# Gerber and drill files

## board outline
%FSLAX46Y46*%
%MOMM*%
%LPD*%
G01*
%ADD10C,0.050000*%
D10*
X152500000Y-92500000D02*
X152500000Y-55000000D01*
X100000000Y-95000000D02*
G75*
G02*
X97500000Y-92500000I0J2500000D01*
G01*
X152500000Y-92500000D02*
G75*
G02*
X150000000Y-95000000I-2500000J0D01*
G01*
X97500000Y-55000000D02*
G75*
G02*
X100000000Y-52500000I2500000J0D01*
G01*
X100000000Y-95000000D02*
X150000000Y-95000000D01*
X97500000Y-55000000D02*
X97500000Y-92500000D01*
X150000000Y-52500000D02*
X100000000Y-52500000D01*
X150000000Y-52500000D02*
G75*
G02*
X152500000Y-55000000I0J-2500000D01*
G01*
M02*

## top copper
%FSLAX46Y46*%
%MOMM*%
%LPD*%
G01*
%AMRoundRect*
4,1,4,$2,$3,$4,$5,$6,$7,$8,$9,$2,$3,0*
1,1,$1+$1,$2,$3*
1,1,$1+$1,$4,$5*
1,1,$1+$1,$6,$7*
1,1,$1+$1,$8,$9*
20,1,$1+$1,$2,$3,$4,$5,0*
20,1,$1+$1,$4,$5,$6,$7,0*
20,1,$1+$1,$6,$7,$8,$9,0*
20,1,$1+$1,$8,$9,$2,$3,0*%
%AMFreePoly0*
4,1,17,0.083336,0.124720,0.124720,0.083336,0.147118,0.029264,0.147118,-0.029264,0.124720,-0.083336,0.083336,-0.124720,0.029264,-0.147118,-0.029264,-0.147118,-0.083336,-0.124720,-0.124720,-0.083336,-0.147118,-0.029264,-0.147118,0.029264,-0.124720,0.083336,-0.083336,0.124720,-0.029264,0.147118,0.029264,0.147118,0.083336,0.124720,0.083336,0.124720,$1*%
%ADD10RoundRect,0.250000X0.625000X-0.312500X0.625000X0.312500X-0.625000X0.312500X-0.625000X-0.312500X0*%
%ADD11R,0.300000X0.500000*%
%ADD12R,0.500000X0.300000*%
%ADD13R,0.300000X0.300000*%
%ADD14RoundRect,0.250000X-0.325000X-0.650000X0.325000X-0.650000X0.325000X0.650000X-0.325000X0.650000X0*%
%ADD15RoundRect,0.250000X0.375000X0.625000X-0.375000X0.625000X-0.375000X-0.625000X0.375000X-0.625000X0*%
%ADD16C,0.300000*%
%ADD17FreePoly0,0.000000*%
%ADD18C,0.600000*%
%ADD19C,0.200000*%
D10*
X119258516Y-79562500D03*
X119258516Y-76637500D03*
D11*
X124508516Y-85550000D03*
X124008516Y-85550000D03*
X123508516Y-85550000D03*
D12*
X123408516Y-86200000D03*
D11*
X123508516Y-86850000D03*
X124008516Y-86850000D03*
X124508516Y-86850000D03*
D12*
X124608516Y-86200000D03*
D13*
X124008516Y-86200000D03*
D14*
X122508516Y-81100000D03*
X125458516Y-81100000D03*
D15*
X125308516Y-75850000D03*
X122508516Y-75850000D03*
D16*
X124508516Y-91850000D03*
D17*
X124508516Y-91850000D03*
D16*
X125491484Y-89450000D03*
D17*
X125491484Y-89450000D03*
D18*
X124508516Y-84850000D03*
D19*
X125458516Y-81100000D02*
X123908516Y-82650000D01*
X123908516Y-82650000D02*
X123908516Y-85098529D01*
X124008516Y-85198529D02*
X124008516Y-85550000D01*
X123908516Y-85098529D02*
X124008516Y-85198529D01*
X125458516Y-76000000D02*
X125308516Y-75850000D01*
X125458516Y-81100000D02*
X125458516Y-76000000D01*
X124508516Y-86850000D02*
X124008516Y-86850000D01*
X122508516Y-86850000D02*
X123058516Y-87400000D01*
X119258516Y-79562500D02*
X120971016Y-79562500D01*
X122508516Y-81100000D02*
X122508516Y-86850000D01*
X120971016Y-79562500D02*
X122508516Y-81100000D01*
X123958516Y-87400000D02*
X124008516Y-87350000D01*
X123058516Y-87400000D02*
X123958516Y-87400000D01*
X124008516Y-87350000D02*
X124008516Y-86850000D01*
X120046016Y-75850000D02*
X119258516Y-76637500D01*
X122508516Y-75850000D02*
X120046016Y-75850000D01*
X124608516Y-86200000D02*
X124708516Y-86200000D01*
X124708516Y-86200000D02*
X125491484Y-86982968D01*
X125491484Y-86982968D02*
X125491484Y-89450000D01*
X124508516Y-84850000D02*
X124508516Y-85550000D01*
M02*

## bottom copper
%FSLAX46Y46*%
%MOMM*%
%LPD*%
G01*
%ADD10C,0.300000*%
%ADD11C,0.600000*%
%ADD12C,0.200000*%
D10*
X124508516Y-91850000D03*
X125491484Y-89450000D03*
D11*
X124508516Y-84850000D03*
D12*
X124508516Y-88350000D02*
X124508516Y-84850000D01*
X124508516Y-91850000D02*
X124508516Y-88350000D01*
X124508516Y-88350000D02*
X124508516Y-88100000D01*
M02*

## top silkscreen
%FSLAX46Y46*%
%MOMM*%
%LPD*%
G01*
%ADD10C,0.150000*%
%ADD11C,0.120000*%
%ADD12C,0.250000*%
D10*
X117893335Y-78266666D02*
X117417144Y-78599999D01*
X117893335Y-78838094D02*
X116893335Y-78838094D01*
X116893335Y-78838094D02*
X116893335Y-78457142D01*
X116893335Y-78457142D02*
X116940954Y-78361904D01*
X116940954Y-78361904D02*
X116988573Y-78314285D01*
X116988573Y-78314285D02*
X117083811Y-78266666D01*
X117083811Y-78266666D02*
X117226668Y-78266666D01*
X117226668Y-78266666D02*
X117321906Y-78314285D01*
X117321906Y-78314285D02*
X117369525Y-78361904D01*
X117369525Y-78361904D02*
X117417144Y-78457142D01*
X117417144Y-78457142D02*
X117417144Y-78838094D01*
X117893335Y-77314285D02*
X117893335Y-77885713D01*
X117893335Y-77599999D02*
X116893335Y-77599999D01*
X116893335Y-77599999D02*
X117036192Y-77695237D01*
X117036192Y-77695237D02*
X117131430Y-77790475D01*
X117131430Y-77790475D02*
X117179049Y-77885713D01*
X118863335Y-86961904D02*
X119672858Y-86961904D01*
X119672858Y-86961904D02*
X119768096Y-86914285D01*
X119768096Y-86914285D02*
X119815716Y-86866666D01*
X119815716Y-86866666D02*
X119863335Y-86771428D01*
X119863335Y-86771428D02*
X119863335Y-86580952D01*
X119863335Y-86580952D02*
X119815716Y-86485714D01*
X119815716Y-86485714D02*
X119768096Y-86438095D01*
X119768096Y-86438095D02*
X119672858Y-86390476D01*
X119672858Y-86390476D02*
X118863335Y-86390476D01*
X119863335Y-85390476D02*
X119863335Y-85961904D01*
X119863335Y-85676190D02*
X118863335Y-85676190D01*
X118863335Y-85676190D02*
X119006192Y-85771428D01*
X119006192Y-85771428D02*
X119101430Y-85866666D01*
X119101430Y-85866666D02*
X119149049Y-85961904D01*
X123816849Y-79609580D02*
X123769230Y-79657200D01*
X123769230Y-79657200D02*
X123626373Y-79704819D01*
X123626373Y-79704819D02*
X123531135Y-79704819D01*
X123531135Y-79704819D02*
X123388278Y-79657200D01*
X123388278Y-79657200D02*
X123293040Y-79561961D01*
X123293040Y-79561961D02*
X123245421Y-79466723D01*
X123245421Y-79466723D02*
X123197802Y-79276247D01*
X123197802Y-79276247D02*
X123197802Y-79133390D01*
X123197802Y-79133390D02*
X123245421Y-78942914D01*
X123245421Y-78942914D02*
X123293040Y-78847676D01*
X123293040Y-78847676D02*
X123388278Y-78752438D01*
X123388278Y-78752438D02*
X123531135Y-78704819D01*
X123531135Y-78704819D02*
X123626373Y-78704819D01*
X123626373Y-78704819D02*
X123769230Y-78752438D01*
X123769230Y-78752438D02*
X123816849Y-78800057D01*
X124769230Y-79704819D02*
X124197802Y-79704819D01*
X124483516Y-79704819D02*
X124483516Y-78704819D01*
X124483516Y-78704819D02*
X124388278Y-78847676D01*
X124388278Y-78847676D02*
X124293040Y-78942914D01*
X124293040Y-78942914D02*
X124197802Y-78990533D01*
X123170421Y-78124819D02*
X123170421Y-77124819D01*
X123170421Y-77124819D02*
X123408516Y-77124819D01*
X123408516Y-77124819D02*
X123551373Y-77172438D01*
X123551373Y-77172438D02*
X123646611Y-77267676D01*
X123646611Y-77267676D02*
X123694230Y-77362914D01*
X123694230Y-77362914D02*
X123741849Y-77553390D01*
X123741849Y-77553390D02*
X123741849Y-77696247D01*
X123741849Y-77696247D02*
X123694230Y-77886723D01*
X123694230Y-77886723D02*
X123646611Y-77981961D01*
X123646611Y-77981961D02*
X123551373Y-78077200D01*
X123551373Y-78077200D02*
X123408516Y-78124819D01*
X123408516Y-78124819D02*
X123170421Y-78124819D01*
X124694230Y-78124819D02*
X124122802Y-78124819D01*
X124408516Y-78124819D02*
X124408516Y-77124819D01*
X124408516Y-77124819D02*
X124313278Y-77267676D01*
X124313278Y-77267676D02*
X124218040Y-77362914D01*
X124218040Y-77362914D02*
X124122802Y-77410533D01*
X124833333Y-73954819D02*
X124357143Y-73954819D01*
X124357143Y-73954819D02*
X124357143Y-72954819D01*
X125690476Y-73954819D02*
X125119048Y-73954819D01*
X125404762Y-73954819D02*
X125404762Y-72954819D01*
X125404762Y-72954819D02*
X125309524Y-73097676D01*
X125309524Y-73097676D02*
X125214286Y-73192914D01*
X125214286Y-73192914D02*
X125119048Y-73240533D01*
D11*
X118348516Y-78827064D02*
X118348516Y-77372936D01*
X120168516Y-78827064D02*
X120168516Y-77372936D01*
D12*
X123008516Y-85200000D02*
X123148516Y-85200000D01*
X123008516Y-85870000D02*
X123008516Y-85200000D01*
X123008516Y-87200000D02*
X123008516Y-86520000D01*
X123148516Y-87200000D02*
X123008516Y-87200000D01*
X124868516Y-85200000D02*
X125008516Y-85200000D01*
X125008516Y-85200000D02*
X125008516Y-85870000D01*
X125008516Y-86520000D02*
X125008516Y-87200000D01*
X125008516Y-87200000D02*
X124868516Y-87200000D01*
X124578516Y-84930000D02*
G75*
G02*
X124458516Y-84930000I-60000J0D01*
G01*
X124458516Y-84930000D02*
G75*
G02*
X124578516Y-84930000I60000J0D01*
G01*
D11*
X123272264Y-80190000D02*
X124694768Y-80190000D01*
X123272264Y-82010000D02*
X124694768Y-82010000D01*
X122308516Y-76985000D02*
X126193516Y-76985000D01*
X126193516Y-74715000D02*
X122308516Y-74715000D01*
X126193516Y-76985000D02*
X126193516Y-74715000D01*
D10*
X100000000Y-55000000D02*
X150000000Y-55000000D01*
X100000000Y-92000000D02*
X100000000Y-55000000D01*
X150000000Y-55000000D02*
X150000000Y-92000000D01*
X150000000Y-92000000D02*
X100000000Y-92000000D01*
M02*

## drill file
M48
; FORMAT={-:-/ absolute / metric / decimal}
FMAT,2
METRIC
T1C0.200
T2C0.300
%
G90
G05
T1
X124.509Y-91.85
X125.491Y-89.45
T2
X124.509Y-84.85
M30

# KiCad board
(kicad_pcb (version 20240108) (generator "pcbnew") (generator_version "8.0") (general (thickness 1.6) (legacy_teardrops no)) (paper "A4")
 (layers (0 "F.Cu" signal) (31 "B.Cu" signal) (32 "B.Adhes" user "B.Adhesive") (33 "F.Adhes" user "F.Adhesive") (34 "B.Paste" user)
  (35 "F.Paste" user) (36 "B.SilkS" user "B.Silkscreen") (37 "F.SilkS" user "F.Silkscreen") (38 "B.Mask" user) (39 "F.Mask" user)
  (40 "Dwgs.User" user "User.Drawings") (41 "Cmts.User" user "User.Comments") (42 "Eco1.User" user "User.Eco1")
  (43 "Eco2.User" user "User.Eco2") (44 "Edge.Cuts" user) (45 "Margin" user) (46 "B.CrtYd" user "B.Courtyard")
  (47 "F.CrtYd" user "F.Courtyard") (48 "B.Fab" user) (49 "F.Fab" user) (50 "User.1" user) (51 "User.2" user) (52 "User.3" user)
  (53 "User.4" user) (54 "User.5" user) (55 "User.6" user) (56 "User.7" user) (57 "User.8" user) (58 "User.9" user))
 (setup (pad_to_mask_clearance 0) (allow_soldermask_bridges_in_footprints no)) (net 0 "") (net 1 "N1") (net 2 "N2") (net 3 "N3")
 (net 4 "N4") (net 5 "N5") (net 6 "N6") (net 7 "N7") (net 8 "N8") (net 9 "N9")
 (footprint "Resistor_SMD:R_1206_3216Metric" (layer "F.Cu") (at 119.258516 78.1 90)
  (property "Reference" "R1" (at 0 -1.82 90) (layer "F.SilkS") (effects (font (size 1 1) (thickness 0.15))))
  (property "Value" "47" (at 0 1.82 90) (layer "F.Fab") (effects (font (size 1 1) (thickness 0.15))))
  (fp_line (start -0.727064 -0.91) (end 0.727064 -0.91) (stroke (width 0.12) (type solid)) (layer "F.SilkS"))
  (fp_line (start -0.727064 0.91) (end 0.727064 0.91) (stroke (width 0.12) (type solid)) (layer "F.SilkS"))
  (pad "1" smd roundrect (at -1.4625 0 90) (size 1.125 1.75) (layers "F.Cu" "F.Paste" "F.Mask") (roundrect_rratio 0.222222) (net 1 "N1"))
  (pad "2" smd roundrect (at 1.4625 0 90) (size 1.125 1.75) (layers "F.Cu" "F.Paste" "F.Mask") (roundrect_rratio 0.222222) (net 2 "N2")))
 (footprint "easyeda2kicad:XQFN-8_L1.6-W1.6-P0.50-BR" (layer "F.Cu") (at 124.008516 86.2 90)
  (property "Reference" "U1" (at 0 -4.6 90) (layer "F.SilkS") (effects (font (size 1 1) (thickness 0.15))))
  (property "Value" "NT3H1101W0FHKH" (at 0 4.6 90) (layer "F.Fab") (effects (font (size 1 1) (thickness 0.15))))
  (fp_line (start 1 -1) (end 1 -0.86) (stroke (width 0.25) (type solid)) (layer "F.SilkS"))
  (fp_line (start 0.33 -1) (end 1 -1) (stroke (width 0.25) (type solid)) (layer "F.SilkS"))
  (fp_line (start -1 -1) (end -0.32 -1) (stroke (width 0.25) (type solid)) (layer "F.SilkS"))
  (fp_line (start -1 -0.86) (end -1 -1) (stroke (width 0.25) (type solid)) (layer "F.SilkS"))
  (fp_line (start 1 0.86) (end 1 1) (stroke (width 0.25) (type solid)) (layer "F.SilkS"))
  (fp_line (start 1 1) (end 0.33 1) (stroke (width 0.25) (type solid)) (layer "F.SilkS"))
  (fp_line (start -0.32 1) (end -1 1) (stroke (width 0.25) (type solid)) (layer "F.SilkS"))
  (fp_line (start -1 1) (end -1 0.86) (stroke (width 0.25) (type solid)) (layer "F.SilkS"))
  (fp_circle (center 1.27 0.51) (end 1.33 0.51) (stroke (width 0.25) (type solid)) (fill none) (layer "F.SilkS"))
  (pad "1" smd rect (at 0.65 0.5 270) (size 0.5 0.3) (layers "F.Cu" "F.Paste" "F.Mask") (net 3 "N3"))
  (pad "2" smd rect (at 0.65 0 270) (size 0.5 0.3) (layers "F.Cu" "F.Paste" "F.Mask") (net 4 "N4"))
  (pad "3" smd rect (at 0.65 -0.5 270) (size 0.5 0.3) (layers "F.Cu" "F.Paste" "F.Mask") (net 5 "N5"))
  (pad "4" smd rect (at 0 -0.6) (size 0.5 0.3) (layers "F.Cu" "F.Paste" "F.Mask") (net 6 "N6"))
  (pad "5" smd rect (at -0.65 -0.5 270) (size 0.5 0.3) (layers "F.Cu" "F.Paste" "F.Mask") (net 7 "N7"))
  (pad "6" smd rect (at -0.65 0 270) (size 0.5 0.3) (layers "F.Cu" "F.Paste" "F.Mask") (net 1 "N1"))
  (pad "7" smd rect (at -0.65 0.5 270) (size 0.5 0.3) (layers "F.Cu" "F.Paste" "F.Mask") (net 1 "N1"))
  (pad "8" smd rect (at 0 0.6) (size 0.5 0.3) (layers "F.Cu" "F.Paste" "F.Mask") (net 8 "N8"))
  (pad "9" smd rect (at 0 0) (size 0.3 0.3) (layers "F.Cu" "F.Paste" "F.Mask") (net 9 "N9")))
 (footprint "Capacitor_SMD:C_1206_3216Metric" (layer "F.Cu") (at 123.983516 81.1)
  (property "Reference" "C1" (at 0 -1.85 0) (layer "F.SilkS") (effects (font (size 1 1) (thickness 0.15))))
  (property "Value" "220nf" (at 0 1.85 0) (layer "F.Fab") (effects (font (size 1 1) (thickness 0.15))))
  (fp_line (start -0.711252 -0.91) (end 0.711252 -0.91) (stroke (width 0.12) (type solid)) (layer "F.SilkS"))
  (fp_line (start -0.711252 0.91) (end 0.711252 0.91) (stroke (width 0.12) (type solid)) (layer "F.SilkS"))
  (pad "1" smd roundrect (at -1.475 0) (size 1.15 1.8) (layers "F.Cu" "F.Paste" "F.Mask") (roundrect_rratio 0.217391) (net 1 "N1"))
  (pad "2" smd roundrect (at 1.475 0) (size 1.15 1.8) (layers "F.Cu" "F.Paste" "F.Mask") (roundrect_rratio 0.217391) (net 4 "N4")))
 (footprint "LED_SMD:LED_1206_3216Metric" (layer "F.Cu") (at 123.908516 75.85 180)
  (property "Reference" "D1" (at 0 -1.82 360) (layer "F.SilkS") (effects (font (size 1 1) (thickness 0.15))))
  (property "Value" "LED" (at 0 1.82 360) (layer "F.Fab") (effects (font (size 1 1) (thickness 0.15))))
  (fp_line (start 1.6 -1.135) (end -2.285 -1.135) (stroke (width 0.12) (type solid)) (layer "F.SilkS"))
  (fp_line (start -2.285 1.135) (end 1.6 1.135) (stroke (width 0.12) (type solid)) (layer "F.SilkS"))
  (fp_line (start -2.285 -1.135) (end -2.285 1.135) (stroke (width 0.12) (type solid)) (layer "F.SilkS"))
  (pad "1" smd roundrect (at -1.4 0 180) (size 1.25 1.75) (layers "F.Cu" "F.Paste" "F.Mask") (roundrect_rratio 0.2) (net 4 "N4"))
  (pad "2" smd roundrect (at 1.4 0 180) (size 1.25 1.75) (layers "F.Cu" "F.Paste" "F.Mask") (roundrect_rratio 0.2) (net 2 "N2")))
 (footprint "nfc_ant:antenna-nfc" (layer "F.Cu") (at 100 55)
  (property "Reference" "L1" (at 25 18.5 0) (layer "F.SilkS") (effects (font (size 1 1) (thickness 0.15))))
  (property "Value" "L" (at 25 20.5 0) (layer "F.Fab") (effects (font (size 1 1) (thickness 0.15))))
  (fp_line (start 0 0) (end 50 0) (stroke (width 0.15) (type solid)) (layer "F.SilkS"))
  (fp_line (start 0 37) (end 0 0) (stroke (width 0.15) (type solid)) (layer "F.SilkS"))
  (fp_line (start 50 0) (end 50 37) (stroke (width 0.15) (type solid)) (layer "F.SilkS"))
  (fp_line (start 50 37) (end 0 37) (stroke (width 0.15) (type solid)) (layer "F.SilkS"))
  (pad "1" thru_hole circle (at 24.508516 36.85) (size 0.3 0.3) (drill 0.2) (layers "*.Cu" "*.Mask") (remove_unused_layers no) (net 3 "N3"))
  (pad "1" smd custom (at 24.508516 36.85) (size 0.3 0.3) (layers "F.Cu") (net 3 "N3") (zone_connect 0) (thermal_bridge_angle 90)
   (options (clearance outline) (anchor circle)) (primitives))
  (pad "2" thru_hole circle (at 25.491484 34.45) (size 0.3 0.3) (drill 0.2) (layers "*.Cu" "*.Mask") (remove_unused_layers no) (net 8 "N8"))
  (pad "2" smd custom (at 25.491484 34.45) (size 0.3 0.3) (layers "F.Cu") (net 8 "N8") (zone_connect 0) (thermal_bridge_angle 90)
   (options (clearance outline) (anchor circle)) (primitives)))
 (gr_line (start 152.5 92.5) (end 152.5 55) (stroke (width 0.05) (type default)) (layer "Edge.Cuts"))
 (gr_arc (start 100 95) (mid 98.232233 94.267767) (end 97.5 92.5) (stroke (width 0.05) (type default)) (layer "Edge.Cuts"))
 (gr_arc (start 152.5 92.5) (mid 151.767767 94.267767) (end 150 95) (stroke (width 0.05) (type default)) (layer "Edge.Cuts"))
 (gr_arc (start 97.5 55) (mid 98.232233 53.232233) (end 100 52.5) (stroke (width 0.05) (type default)) (layer "Edge.Cuts"))
 (gr_line (start 100 95) (end 150 95) (stroke (width 0.05) (type default)) (layer "Edge.Cuts"))
 (gr_line (start 97.5 55) (end 97.5 92.5) (stroke (width 0.05) (type default)) (layer "Edge.Cuts"))
 (gr_line (start 150 52.5) (end 100 52.5) (stroke (width 0.05) (type default)) (layer "Edge.Cuts"))
 (gr_arc (start 150 52.5) (mid 151.767767 53.232233) (end 152.5 55) (stroke (width 0.05) (type default)) (layer "Edge.Cuts"))
 (segment (start 125.458516 81.1) (end 123.908516 82.65) (width 0.2) (layer "F.Cu") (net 4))
 (segment (start 123.908516 82.65) (end 123.908516 85.098529) (width 0.2) (layer "F.Cu") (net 4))
 (segment (start 124.008516 85.198529) (end 124.008516 85.55) (width 0.2) (layer "F.Cu") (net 4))
 (segment (start 123.908516 85.098529) (end 124.008516 85.198529) (width 0.2) (layer "F.Cu") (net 4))
 (segment (start 125.458516 76) (end 125.308516 75.85) (width 0.2) (layer "F.Cu") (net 4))
 (segment (start 125.458516 81.1) (end 125.458516 76) (width 0.2) (layer "F.Cu") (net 4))
 (segment (start 124.508516 86.85) (end 124.008516 86.85) (width 0.2) (layer "F.Cu") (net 1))
 (segment (start 122.508516 86.85) (end 123.058516 87.4) (width 0.2) (layer "F.Cu") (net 1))
 (segment (start 119.258516 79.5625) (end 120.971016 79.5625) (width 0.2) (layer "F.Cu") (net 1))
 (segment (start 122.508516 81.1) (end 122.508516 86.85) (width 0.2) (layer "F.Cu") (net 1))
 (segment (start 120.971016 79.5625) (end 122.508516 81.1) (width 0.2) (layer "F.Cu") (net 1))
 (segment (start 123.958516 87.4) (end 124.008516 87.35) (width 0.2) (layer "F.Cu") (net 1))
 (segment (start 123.058516 87.4) (end 123.958516 87.4) (width 0.2) (layer "F.Cu") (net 1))
 (segment (start 124.008516 87.35) (end 124.008516 86.85) (width 0.2) (layer "F.Cu") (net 1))
 (segment (start 120.046016 75.85) (end 119.258516 76.6375) (width 0.2) (layer "F.Cu") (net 2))
 (segment (start 122.508516 75.85) (end 120.046016 75.85) (width 0.2) (layer "F.Cu") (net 2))
 (segment (start 124.608516 86.2) (end 124.708516 86.2) (width 0.2) (layer "F.Cu") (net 8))
 (segment (start 124.708516 86.2) (end 125.491484 86.982968) (width 0.2) (layer "F.Cu") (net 8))
 (segment (start 125.491484 86.982968) (end 125.491484 89.45) (width 0.2) (layer "F.Cu") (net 8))
 (segment (start 124.508516 84.85) (end 124.508516 85.55) (width 0.2) (layer "F.Cu") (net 3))
 (via (at 124.508516 84.85) (size 0.6) (drill 0.3) (layers "F.Cu" "B.Cu") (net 3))
 (segment (start 124.508516 88.35) (end 124.508516 84.85) (width 0.2) (layer "B.Cu") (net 3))
 (segment (start 124.508516 91.85) (end 124.508516 88.35) (width 0.2) (layer "B.Cu") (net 3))
 (segment (start 124.508516 88.35) (end 124.508516 88.1) (width 0.2) (layer "B.Cu") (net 3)))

